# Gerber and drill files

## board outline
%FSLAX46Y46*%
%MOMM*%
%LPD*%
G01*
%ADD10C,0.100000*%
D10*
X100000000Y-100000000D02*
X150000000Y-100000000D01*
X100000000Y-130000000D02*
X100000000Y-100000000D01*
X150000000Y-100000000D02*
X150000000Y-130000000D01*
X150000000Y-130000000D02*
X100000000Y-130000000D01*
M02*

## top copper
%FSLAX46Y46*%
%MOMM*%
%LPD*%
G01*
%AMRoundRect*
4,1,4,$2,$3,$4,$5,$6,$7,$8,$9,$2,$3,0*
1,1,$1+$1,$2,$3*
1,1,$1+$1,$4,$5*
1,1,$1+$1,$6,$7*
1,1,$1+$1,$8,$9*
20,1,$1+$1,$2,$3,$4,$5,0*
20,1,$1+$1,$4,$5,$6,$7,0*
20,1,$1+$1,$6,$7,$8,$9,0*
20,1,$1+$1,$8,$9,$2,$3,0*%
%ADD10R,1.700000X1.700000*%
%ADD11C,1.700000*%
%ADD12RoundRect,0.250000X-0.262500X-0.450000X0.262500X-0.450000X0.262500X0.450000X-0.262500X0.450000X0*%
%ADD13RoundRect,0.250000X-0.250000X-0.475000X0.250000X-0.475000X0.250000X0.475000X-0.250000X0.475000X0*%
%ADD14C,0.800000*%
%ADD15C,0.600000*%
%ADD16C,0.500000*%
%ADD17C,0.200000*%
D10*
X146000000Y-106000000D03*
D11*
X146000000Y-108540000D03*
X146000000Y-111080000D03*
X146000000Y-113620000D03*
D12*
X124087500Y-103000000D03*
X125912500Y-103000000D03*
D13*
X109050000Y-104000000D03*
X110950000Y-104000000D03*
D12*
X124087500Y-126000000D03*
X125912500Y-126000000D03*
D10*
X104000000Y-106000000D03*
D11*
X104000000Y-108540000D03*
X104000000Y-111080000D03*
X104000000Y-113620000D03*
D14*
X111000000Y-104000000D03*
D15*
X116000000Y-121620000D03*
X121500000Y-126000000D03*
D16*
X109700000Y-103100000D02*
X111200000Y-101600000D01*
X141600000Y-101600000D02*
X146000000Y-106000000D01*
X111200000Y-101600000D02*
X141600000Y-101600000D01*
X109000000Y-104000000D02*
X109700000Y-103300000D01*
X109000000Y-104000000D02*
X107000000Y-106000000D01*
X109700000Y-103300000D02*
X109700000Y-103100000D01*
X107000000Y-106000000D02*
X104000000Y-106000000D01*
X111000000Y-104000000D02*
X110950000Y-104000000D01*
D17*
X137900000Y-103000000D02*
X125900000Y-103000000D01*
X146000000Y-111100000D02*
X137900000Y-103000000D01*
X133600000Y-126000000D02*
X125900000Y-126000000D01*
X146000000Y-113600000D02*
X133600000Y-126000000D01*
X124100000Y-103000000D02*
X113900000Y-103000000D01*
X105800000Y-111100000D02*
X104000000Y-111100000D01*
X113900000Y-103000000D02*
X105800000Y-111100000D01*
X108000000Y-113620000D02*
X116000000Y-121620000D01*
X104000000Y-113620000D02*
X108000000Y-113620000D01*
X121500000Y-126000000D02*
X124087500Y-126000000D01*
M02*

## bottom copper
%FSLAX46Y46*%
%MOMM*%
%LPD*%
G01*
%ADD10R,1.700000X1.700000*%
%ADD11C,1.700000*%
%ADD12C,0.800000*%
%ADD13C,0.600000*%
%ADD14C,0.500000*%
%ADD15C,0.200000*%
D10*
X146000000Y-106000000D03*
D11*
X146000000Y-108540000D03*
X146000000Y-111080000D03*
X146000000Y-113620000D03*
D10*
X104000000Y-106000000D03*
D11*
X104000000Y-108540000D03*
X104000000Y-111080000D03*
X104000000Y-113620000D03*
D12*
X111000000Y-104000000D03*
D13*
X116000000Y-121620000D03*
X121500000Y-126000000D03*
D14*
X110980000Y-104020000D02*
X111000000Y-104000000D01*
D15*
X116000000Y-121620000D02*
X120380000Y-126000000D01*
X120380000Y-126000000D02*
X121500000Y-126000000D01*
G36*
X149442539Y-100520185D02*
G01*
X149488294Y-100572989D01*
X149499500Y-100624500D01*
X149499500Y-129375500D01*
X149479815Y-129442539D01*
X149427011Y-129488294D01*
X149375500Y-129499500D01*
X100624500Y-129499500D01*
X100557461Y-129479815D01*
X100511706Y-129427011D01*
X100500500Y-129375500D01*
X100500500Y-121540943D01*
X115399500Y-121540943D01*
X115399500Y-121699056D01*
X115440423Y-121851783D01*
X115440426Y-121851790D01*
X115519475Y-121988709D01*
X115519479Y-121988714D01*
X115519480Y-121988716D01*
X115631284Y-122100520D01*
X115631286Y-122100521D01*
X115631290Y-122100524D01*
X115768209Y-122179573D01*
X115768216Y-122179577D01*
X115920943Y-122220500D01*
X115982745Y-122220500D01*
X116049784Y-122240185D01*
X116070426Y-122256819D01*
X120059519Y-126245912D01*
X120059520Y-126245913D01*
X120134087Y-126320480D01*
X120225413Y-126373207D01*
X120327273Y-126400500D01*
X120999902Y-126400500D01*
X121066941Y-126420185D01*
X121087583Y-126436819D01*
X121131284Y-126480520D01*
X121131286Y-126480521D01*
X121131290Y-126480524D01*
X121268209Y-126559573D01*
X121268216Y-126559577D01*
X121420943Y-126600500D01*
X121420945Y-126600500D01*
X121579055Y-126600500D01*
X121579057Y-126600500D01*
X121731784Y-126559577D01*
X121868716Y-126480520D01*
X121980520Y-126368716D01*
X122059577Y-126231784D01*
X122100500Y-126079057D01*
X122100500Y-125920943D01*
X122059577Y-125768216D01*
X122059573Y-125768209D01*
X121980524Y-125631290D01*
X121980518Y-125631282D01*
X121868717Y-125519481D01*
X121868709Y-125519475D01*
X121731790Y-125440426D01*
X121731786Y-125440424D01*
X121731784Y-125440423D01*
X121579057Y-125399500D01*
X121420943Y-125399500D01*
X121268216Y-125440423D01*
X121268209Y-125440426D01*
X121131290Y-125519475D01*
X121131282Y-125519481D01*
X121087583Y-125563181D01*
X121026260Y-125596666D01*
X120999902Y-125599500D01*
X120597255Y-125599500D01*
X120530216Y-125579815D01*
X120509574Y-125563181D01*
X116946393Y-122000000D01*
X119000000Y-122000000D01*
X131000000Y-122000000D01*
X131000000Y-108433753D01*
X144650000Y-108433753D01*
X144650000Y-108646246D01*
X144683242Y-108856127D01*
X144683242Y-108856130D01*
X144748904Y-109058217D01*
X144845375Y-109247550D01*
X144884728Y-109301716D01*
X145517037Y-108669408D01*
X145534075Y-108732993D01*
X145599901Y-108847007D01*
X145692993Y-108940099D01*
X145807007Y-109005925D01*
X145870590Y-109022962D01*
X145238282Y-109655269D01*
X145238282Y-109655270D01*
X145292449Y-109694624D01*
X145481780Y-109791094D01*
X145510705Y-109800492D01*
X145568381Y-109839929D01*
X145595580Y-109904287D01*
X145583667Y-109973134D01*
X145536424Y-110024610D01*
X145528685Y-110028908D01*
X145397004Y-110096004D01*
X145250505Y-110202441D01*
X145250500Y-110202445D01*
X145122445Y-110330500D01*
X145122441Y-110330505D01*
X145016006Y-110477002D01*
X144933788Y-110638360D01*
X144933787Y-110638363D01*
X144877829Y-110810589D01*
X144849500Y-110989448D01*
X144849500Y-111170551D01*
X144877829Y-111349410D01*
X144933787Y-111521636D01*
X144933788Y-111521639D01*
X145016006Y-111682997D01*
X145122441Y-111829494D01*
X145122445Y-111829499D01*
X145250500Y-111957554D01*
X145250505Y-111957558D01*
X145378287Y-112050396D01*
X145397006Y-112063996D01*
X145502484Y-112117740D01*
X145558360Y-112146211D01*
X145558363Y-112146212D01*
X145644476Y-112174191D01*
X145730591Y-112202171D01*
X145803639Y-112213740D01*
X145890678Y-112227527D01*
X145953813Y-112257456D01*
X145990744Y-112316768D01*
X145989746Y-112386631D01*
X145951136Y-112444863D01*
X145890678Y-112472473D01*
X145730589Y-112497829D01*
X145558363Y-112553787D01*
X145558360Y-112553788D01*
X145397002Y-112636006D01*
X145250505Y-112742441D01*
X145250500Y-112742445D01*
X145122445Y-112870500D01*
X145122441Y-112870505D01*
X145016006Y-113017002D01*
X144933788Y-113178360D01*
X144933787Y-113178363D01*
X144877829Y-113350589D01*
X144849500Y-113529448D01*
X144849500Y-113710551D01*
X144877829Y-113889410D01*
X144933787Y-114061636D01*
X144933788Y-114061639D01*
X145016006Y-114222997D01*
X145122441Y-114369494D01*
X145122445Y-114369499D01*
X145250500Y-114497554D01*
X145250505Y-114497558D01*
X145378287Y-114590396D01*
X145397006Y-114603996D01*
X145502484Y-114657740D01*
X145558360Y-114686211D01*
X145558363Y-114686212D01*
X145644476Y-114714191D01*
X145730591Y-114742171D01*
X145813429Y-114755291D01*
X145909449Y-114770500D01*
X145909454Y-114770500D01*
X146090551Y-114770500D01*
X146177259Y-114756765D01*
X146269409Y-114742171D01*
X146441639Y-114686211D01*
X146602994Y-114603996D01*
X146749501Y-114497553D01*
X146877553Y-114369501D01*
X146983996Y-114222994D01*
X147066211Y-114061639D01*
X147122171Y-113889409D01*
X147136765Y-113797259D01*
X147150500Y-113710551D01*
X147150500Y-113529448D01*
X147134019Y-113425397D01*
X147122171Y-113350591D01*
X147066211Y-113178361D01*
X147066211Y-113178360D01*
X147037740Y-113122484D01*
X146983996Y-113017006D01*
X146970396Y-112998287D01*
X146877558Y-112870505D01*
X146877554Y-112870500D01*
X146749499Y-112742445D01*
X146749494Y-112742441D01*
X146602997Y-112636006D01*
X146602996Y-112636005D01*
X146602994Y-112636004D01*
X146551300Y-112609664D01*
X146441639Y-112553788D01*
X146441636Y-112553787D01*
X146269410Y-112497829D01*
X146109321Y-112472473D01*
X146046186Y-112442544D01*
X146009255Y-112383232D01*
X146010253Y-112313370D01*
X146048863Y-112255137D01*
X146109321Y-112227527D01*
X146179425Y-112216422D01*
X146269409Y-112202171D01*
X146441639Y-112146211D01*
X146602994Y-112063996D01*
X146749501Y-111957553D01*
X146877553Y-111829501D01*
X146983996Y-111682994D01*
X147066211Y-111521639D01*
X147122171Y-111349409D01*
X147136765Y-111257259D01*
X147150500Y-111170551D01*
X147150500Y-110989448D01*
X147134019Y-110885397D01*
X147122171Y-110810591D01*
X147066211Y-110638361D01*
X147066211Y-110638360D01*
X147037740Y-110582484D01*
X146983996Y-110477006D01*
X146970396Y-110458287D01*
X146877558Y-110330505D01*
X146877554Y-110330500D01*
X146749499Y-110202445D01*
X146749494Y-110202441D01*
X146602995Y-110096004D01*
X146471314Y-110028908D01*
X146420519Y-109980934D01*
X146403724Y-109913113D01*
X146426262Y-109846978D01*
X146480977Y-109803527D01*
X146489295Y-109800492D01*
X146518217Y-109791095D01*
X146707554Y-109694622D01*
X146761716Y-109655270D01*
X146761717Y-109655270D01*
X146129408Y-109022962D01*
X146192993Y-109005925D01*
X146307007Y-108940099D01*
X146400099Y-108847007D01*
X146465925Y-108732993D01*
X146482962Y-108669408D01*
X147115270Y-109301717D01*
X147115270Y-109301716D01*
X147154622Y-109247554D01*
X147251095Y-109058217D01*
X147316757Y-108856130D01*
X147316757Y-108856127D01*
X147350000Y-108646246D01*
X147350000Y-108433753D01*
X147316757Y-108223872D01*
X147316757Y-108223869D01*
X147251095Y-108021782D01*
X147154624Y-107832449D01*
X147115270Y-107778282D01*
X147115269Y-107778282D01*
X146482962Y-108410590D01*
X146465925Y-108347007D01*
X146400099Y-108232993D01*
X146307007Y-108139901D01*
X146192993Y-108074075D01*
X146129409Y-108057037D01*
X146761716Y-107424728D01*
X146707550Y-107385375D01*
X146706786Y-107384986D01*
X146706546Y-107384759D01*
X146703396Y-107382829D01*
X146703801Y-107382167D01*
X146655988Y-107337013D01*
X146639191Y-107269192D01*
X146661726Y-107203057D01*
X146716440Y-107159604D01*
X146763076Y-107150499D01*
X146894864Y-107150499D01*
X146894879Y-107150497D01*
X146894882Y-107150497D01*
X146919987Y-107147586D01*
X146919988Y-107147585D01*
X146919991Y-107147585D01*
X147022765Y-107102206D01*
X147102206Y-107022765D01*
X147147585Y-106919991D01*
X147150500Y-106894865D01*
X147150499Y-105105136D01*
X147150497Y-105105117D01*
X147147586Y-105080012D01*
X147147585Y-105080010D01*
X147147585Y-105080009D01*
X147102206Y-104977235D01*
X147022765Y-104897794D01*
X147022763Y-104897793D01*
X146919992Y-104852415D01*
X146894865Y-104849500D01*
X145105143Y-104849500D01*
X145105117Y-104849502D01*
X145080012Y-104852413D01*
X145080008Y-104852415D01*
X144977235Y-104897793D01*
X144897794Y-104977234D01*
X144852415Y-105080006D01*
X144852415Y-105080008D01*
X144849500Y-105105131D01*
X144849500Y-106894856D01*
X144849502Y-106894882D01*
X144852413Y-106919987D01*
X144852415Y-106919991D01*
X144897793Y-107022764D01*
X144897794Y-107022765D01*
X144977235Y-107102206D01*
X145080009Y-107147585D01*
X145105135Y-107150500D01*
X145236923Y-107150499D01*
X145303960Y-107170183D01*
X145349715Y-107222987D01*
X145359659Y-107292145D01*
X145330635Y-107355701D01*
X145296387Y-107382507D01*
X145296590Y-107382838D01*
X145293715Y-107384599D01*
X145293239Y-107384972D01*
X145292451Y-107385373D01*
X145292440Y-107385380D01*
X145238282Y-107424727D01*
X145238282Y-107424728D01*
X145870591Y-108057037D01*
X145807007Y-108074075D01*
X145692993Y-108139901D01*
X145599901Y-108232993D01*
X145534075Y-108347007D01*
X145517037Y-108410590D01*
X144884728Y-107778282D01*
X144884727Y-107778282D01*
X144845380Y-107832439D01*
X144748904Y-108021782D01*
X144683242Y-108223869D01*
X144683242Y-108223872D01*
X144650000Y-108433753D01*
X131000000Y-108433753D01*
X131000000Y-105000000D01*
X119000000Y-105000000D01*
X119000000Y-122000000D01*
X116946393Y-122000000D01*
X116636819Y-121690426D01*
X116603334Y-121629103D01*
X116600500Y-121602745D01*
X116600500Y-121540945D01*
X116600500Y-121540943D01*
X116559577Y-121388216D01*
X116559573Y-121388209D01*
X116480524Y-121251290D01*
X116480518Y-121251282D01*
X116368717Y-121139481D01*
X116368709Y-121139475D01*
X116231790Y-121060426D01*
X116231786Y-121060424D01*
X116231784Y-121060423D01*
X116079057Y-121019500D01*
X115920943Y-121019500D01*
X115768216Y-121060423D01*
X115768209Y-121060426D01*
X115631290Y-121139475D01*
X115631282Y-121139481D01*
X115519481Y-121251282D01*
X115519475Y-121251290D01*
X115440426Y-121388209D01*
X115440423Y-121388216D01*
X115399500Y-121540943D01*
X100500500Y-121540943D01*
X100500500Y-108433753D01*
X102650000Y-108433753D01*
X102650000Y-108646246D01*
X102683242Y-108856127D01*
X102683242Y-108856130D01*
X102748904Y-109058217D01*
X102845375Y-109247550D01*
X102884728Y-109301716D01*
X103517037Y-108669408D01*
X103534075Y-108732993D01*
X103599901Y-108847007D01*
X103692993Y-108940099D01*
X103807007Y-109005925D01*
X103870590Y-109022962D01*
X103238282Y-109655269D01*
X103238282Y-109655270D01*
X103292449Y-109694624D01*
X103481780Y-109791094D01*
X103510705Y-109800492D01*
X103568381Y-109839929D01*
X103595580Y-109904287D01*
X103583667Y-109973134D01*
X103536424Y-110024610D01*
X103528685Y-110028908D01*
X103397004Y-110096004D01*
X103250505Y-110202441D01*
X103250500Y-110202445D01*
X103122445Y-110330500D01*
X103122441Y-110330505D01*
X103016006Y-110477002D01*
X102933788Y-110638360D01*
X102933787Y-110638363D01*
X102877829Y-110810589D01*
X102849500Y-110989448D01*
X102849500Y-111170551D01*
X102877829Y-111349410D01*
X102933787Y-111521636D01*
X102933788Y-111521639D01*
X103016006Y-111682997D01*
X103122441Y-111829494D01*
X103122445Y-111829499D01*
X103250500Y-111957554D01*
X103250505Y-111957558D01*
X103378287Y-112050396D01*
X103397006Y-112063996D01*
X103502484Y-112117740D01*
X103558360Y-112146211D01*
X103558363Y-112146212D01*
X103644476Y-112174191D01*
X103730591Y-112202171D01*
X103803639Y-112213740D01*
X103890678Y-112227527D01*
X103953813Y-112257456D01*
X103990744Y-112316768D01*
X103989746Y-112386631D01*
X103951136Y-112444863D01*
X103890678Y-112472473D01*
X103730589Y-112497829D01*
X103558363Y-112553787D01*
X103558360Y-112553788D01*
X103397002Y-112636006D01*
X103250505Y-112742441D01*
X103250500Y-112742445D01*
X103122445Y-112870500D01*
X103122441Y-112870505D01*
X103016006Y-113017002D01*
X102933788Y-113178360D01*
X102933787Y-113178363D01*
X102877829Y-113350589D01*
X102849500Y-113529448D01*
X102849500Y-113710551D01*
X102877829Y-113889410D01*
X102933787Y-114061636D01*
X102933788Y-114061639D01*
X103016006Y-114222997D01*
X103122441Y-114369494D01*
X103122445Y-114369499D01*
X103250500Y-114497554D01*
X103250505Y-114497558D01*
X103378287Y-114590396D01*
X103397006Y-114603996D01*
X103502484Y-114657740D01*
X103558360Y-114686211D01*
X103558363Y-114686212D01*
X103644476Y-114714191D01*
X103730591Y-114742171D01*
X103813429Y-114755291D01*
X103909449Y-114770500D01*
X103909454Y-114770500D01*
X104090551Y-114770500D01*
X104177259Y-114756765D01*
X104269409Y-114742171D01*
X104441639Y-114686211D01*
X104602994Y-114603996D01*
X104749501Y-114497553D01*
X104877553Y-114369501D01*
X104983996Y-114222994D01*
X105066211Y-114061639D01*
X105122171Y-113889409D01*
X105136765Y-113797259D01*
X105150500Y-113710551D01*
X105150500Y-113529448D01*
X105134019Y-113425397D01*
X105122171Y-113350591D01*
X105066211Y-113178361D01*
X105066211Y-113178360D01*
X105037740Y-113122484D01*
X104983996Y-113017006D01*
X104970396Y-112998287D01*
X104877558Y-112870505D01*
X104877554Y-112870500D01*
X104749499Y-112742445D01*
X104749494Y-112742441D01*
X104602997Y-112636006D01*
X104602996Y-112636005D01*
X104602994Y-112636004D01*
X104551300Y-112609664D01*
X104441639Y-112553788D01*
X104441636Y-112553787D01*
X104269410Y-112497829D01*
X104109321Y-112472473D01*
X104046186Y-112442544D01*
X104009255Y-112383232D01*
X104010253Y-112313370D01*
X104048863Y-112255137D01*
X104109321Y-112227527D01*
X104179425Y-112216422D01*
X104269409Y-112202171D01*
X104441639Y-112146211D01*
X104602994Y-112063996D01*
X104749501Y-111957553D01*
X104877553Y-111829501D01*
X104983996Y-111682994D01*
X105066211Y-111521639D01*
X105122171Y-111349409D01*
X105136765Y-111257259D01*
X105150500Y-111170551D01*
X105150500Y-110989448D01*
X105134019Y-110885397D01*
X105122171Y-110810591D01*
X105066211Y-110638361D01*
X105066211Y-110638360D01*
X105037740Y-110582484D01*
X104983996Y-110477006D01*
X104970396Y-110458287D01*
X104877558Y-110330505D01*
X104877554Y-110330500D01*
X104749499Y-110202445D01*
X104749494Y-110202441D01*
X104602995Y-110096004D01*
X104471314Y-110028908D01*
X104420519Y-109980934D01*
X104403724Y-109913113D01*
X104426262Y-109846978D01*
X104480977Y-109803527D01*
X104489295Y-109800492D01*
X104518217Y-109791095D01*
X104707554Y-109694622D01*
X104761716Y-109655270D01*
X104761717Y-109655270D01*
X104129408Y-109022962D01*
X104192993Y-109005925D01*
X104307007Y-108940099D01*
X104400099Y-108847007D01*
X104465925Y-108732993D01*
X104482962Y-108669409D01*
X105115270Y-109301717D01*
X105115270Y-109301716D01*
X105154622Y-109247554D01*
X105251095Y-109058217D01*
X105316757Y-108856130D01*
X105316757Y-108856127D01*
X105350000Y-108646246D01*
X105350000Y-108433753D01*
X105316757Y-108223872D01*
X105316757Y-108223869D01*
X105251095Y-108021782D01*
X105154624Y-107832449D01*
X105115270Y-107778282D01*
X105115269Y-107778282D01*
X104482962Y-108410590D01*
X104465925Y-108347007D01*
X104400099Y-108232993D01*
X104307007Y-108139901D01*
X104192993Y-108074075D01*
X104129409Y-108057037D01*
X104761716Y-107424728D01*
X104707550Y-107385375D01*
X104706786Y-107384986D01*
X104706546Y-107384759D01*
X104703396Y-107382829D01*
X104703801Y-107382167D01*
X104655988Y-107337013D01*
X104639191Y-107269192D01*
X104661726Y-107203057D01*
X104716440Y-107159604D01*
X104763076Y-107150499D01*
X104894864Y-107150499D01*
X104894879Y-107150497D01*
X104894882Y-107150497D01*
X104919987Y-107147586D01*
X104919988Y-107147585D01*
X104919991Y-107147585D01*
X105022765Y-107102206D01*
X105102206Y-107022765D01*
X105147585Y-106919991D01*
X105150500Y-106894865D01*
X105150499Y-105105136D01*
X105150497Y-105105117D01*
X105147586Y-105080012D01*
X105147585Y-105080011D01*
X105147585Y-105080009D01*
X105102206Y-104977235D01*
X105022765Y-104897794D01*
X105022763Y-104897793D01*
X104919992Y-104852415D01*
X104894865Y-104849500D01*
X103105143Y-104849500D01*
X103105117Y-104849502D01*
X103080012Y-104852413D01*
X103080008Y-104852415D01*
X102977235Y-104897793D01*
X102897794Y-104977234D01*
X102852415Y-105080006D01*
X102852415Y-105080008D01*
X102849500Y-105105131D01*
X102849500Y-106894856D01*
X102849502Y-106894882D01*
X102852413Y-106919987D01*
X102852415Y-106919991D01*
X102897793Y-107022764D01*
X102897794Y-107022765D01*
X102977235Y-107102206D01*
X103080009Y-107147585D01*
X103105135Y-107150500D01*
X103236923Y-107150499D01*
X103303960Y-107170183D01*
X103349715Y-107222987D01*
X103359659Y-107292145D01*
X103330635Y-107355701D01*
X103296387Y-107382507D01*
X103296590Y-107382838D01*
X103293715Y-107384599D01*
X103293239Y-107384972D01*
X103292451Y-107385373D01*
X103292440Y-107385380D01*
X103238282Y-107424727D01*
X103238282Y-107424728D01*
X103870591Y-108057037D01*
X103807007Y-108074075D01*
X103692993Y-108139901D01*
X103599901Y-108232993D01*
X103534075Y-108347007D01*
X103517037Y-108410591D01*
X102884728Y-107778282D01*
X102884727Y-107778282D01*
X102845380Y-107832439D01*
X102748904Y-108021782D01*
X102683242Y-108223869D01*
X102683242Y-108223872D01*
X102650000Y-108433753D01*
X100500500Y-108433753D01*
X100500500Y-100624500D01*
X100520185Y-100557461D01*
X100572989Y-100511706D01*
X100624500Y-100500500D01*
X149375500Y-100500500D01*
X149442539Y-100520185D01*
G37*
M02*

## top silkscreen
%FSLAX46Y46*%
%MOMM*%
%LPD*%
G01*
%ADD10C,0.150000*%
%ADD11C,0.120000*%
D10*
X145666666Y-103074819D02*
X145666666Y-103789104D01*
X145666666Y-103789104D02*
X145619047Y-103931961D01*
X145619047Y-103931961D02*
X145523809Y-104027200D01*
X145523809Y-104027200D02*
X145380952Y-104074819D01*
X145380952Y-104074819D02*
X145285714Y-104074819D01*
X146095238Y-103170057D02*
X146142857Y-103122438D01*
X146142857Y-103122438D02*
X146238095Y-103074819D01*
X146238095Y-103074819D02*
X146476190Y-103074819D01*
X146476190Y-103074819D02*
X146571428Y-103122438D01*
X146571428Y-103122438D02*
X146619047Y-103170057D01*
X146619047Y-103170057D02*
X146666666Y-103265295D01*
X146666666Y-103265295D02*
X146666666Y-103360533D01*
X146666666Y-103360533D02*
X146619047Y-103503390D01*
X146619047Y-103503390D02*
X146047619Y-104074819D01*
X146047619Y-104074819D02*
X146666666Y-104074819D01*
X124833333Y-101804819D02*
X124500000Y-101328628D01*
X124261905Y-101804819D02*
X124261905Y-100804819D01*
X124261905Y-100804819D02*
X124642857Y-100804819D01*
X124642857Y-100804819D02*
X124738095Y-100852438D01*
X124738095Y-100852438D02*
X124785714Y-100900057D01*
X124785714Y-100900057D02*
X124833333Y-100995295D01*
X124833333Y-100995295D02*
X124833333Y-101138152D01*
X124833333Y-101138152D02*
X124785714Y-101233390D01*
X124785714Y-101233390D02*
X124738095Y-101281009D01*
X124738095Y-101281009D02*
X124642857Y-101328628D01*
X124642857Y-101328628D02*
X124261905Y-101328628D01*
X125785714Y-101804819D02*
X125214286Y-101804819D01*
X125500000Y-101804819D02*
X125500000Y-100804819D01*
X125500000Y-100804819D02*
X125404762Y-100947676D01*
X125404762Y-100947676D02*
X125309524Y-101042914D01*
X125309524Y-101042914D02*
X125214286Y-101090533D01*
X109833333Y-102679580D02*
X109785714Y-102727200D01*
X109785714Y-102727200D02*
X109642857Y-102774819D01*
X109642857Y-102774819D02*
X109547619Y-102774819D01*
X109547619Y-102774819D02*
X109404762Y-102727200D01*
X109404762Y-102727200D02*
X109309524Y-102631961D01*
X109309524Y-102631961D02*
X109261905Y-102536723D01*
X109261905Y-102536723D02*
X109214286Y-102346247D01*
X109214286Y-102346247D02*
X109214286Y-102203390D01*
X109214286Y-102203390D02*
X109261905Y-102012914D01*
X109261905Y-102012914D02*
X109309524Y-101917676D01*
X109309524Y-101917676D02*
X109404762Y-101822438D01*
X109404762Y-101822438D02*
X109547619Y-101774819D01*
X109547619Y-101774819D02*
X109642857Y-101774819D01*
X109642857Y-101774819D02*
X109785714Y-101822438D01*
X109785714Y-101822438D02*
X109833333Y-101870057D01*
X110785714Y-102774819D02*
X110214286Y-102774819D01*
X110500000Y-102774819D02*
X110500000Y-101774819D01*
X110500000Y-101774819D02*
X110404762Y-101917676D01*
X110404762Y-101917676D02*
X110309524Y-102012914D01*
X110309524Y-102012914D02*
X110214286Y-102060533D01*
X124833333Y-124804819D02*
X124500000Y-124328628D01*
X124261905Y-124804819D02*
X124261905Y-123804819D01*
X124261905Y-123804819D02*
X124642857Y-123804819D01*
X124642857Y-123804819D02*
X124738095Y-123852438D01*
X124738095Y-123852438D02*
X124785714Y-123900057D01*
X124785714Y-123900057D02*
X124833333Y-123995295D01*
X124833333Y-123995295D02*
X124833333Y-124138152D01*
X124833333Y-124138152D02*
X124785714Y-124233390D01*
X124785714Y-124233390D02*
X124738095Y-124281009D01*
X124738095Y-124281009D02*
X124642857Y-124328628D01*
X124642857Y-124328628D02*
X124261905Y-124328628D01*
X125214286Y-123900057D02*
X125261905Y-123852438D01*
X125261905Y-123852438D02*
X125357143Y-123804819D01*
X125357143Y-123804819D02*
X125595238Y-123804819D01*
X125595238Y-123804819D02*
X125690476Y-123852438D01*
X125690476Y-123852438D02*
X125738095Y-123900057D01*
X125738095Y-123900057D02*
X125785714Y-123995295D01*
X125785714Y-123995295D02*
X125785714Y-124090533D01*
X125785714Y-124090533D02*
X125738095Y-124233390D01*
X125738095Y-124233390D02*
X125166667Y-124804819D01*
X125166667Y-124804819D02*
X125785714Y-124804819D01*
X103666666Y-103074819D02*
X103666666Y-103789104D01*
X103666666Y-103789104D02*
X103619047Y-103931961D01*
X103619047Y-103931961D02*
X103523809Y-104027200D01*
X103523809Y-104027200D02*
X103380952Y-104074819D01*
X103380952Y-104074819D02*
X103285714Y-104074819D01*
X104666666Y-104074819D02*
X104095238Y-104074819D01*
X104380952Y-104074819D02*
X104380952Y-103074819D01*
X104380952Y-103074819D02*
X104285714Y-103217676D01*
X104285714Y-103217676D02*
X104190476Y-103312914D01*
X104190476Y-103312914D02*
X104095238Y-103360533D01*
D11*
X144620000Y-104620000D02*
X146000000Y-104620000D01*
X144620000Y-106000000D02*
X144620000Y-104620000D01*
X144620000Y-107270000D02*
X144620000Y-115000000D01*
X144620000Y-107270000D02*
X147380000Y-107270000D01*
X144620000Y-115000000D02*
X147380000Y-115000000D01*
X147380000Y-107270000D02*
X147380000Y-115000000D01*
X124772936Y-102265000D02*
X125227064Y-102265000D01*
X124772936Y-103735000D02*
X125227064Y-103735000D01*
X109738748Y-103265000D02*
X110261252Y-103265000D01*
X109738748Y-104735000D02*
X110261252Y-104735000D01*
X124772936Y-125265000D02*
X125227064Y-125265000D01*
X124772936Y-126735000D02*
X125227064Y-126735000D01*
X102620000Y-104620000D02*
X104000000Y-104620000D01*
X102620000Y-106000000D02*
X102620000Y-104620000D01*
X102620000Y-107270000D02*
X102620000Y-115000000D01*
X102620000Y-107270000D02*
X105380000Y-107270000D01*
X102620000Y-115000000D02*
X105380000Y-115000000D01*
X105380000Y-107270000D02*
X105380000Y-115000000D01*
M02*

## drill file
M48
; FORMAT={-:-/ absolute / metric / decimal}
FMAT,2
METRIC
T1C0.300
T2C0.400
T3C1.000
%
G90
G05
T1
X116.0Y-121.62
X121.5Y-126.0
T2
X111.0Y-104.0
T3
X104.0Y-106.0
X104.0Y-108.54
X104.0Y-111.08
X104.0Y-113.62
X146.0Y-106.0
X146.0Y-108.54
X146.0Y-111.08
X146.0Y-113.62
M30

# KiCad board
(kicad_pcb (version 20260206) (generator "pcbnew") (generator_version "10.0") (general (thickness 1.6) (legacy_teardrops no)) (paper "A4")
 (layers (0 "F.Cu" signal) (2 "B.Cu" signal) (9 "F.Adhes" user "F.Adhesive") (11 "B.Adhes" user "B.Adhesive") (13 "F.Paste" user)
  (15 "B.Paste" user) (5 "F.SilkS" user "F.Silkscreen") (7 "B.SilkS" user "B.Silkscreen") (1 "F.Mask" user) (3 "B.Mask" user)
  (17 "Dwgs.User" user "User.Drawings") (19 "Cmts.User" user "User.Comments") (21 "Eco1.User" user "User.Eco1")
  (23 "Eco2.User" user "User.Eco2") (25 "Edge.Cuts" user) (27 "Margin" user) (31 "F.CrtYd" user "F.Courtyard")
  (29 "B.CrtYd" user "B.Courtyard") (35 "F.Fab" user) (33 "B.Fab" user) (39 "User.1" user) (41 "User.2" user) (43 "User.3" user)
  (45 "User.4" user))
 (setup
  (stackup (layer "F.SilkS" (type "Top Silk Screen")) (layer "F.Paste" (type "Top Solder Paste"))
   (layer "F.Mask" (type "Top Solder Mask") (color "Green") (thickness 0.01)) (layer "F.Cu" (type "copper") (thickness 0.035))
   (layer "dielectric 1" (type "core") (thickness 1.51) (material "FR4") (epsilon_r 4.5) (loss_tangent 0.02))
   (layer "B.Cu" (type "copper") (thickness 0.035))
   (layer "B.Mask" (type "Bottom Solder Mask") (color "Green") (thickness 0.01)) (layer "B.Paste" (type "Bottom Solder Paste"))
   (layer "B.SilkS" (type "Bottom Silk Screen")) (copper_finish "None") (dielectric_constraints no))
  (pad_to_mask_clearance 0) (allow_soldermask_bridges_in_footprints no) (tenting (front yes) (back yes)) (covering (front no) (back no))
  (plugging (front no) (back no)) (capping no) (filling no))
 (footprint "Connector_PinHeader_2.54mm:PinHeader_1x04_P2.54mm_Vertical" (layer "F.Cu") (at 146 106)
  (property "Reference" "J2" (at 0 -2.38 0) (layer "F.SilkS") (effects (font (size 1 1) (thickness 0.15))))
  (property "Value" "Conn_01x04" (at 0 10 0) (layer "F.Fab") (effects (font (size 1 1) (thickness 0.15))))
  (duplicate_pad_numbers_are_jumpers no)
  (fp_line (start -1.38 -1.38) (end 0 -1.38) (stroke (width 0.12) (type solid)) (layer "F.SilkS"))
  (fp_line (start -1.38 0) (end -1.38 -1.38) (stroke (width 0.12) (type solid)) (layer "F.SilkS"))
  (fp_line (start -1.38 1.27) (end -1.38 9) (stroke (width 0.12) (type solid)) (layer "F.SilkS"))
  (fp_line (start -1.38 1.27) (end 1.38 1.27) (stroke (width 0.12) (type solid)) (layer "F.SilkS"))
  (fp_line (start -1.38 9) (end 1.38 9) (stroke (width 0.12) (type solid)) (layer "F.SilkS"))
  (fp_line (start 1.38 1.27) (end 1.38 9) (stroke (width 0.12) (type solid)) (layer "F.SilkS"))
  (pad "1" thru_hole rect (at 0 0) (size 1.7 1.7) (drill 1) (layers "*.Cu" "*.Mask") (remove_unused_layers no) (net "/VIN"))
  (pad "2" thru_hole circle (at 0 2.54) (size 1.7 1.7) (drill 1) (layers "*.Cu" "*.Mask") (remove_unused_layers no) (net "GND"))
  (pad "3" thru_hole circle (at 0 5.08) (size 1.7 1.7) (drill 1) (layers "*.Cu" "*.Mask") (remove_unused_layers no) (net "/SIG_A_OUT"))
  (pad "4" thru_hole circle (at 0 7.62) (size 1.7 1.7) (drill 1) (layers "*.Cu" "*.Mask") (remove_unused_layers no) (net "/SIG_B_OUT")))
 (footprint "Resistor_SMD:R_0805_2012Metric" (layer "F.Cu") (at 125 103)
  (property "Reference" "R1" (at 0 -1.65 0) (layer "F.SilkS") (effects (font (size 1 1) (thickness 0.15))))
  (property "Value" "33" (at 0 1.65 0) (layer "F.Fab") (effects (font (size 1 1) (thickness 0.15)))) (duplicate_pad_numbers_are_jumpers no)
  (fp_line (start -0.227064 -0.735) (end 0.227064 -0.735) (stroke (width 0.12) (type solid)) (layer "F.SilkS"))
  (fp_line (start -0.227064 0.735) (end 0.227064 0.735) (stroke (width 0.12) (type solid)) (layer "F.SilkS"))
  (pad "1" smd roundrect (at -0.9125 0) (size 1.025 1.4) (layers "F.Cu" "F.Mask" "F.Paste") (roundrect_rratio 0.243902) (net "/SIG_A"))
  (pad "2" smd roundrect (at 0.9125 0) (size 1.025 1.4) (layers "F.Cu" "F.Mask" "F.Paste") (roundrect_rratio 0.243902) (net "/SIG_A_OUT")))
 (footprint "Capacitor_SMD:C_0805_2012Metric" (layer "F.Cu") (at 110 104)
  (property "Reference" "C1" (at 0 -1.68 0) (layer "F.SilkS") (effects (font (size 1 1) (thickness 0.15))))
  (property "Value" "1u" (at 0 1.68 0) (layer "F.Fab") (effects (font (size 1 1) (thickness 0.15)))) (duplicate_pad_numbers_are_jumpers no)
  (fp_line (start -0.261252 -0.735) (end 0.261252 -0.735) (stroke (width 0.12) (type solid)) (layer "F.SilkS"))
  (fp_line (start -0.261252 0.735) (end 0.261252 0.735) (stroke (width 0.12) (type solid)) (layer "F.SilkS"))
  (pad "1" smd roundrect (at -0.95 0) (size 1 1.45) (layers "F.Cu" "F.Mask" "F.Paste") (roundrect_rratio 0.25) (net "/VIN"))
  (pad "2" smd roundrect (at 0.95 0) (size 1 1.45) (layers "F.Cu" "F.Mask" "F.Paste") (roundrect_rratio 0.25) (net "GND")))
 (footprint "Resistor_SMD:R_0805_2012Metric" (layer "F.Cu") (at 125 126)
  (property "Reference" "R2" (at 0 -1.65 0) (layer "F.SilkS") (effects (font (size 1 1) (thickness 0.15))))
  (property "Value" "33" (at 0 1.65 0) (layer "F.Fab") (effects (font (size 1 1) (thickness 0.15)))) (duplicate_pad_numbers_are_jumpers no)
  (fp_line (start -0.227064 -0.735) (end 0.227064 -0.735) (stroke (width 0.12) (type solid)) (layer "F.SilkS"))
  (fp_line (start -0.227064 0.735) (end 0.227064 0.735) (stroke (width 0.12) (type solid)) (layer "F.SilkS"))
  (pad "1" smd roundrect (at -0.9125 0) (size 1.025 1.4) (layers "F.Cu" "F.Mask" "F.Paste") (roundrect_rratio 0.243902) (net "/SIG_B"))
  (pad "2" smd roundrect (at 0.9125 0) (size 1.025 1.4) (layers "F.Cu" "F.Mask" "F.Paste") (roundrect_rratio 0.243902) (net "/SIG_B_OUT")))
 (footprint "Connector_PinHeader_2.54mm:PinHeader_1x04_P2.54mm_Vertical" (layer "F.Cu") (at 104 106)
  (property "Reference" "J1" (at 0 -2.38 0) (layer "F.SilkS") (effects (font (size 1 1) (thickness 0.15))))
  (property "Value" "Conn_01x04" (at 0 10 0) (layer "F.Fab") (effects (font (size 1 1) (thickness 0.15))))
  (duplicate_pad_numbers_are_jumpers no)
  (fp_line (start -1.38 -1.38) (end 0 -1.38) (stroke (width 0.12) (type solid)) (layer "F.SilkS"))
  (fp_line (start -1.38 0) (end -1.38 -1.38) (stroke (width 0.12) (type solid)) (layer "F.SilkS"))
  (fp_line (start -1.38 1.27) (end -1.38 9) (stroke (width 0.12) (type solid)) (layer "F.SilkS"))
  (fp_line (start -1.38 1.27) (end 1.38 1.27) (stroke (width 0.12) (type solid)) (layer "F.SilkS"))
  (fp_line (start -1.38 9) (end 1.38 9) (stroke (width 0.12) (type solid)) (layer "F.SilkS"))
  (fp_line (start 1.38 1.27) (end 1.38 9) (stroke (width 0.12) (type solid)) (layer "F.SilkS"))
  (pad "1" thru_hole rect (at 0 0) (size 1.7 1.7) (drill 1) (layers "*.Cu" "*.Mask") (remove_unused_layers no) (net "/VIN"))
  (pad "2" thru_hole circle (at 0 2.54) (size 1.7 1.7) (drill 1) (layers "*.Cu" "*.Mask") (remove_unused_layers no) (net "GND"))
  (pad "3" thru_hole circle (at 0 5.08) (size 1.7 1.7) (drill 1) (layers "*.Cu" "*.Mask") (remove_unused_layers no) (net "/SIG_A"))
  (pad "4" thru_hole circle (at 0 7.62) (size 1.7 1.7) (drill 1) (layers "*.Cu" "*.Mask") (remove_unused_layers no) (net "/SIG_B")))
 (gr_line (start 100 100) (end 150 100) (stroke (width 0.1) (type default)) (layer "Edge.Cuts"))
 (gr_line (start 100 130) (end 100 100) (stroke (width 0.1) (type default)) (layer "Edge.Cuts"))
 (gr_line (start 150 100) (end 150 130) (stroke (width 0.1) (type default)) (layer "Edge.Cuts"))
 (gr_line (start 150 130) (end 100 130) (stroke (width 0.1) (type default)) (layer "Edge.Cuts"))
 (segment (start 109.7 103.1) (end 111.2 101.6) (width 0.5) (layer "F.Cu") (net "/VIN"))
 (segment (start 141.6 101.6) (end 146 106) (width 0.5) (layer "F.Cu") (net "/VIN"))
 (segment (start 111.2 101.6) (end 141.6 101.6) (width 0.5) (layer "F.Cu") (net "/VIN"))
 (segment (start 109 104) (end 109.7 103.3) (width 0.5) (layer "F.Cu") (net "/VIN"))
 (segment (start 109 104) (end 107 106) (width 0.5) (layer "F.Cu") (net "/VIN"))
 (segment (start 109.7 103.3) (end 109.7 103.1) (width 0.5) (layer "F.Cu") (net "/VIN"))
 (segment (start 107 106) (end 104 106) (width 0.5) (layer "F.Cu") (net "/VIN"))
 (segment (start 111 104) (end 110.95 104) (width 0.5) (layer "F.Cu") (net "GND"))
 (via (at 111 104) (size 0.8) (drill 0.4) (layers "F.Cu" "B.Cu") (capping yes) (filling yes) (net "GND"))
 (segment (start 110.98 104.02) (end 111 104) (width 0.5) (layer "B.Cu") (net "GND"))
 (segment (start 137.9 103) (end 125.9 103) (width 0.2) (layer "F.Cu") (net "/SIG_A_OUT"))
 (segment (start 146 111.1) (end 137.9 103) (width 0.2) (layer "F.Cu") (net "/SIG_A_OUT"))
 (segment (start 133.6 126) (end 125.9 126) (width 0.2) (layer "F.Cu") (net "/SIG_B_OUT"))
 (segment (start 146 113.6) (end 133.6 126) (width 0.2) (layer "F.Cu") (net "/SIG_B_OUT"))
 (segment (start 124.1 103) (end 113.9 103) (width 0.2) (layer "F.Cu") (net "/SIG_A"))
 (segment (start 105.8 111.1) (end 104 111.1) (width 0.2) (layer "F.Cu") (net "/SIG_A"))
 (segment (start 113.9 103) (end 105.8 111.1) (width 0.2) (layer "F.Cu") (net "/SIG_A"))
 (segment (start 108 113.62) (end 116 121.62) (width 0.2) (locked yes) (layer "F.Cu") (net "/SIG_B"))
 (segment (start 104 113.62) (end 108 113.62) (width 0.2) (locked yes) (layer "F.Cu") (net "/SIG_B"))
 (segment (start 121.5 126) (end 124.0875 126) (width 0.2) (locked yes) (layer "F.Cu") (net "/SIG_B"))
 (via (at 116 121.62) (size 0.6) (drill 0.3) (layers "F.Cu" "B.Cu") (locked yes) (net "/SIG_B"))
 (via (at 121.5 126) (size 0.6) (drill 0.3) (layers "F.Cu" "B.Cu") (locked yes) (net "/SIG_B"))
 (segment (start 116 121.62) (end 120.38 126) (width 0.2) (locked yes) (layer "B.Cu") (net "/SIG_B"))
 (segment (start 120.38 126) (end 121.5 126) (width 0.2) (locked yes) (layer "B.Cu") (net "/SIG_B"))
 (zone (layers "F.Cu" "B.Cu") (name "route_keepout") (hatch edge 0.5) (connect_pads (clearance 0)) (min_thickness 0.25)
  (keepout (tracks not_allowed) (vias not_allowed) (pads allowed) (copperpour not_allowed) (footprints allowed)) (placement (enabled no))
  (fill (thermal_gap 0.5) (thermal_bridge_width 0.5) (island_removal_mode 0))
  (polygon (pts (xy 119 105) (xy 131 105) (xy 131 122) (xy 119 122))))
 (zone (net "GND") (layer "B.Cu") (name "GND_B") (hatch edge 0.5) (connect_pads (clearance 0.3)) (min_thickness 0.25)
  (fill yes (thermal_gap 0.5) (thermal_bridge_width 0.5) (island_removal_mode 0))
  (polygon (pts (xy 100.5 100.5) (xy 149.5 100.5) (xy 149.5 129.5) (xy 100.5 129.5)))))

